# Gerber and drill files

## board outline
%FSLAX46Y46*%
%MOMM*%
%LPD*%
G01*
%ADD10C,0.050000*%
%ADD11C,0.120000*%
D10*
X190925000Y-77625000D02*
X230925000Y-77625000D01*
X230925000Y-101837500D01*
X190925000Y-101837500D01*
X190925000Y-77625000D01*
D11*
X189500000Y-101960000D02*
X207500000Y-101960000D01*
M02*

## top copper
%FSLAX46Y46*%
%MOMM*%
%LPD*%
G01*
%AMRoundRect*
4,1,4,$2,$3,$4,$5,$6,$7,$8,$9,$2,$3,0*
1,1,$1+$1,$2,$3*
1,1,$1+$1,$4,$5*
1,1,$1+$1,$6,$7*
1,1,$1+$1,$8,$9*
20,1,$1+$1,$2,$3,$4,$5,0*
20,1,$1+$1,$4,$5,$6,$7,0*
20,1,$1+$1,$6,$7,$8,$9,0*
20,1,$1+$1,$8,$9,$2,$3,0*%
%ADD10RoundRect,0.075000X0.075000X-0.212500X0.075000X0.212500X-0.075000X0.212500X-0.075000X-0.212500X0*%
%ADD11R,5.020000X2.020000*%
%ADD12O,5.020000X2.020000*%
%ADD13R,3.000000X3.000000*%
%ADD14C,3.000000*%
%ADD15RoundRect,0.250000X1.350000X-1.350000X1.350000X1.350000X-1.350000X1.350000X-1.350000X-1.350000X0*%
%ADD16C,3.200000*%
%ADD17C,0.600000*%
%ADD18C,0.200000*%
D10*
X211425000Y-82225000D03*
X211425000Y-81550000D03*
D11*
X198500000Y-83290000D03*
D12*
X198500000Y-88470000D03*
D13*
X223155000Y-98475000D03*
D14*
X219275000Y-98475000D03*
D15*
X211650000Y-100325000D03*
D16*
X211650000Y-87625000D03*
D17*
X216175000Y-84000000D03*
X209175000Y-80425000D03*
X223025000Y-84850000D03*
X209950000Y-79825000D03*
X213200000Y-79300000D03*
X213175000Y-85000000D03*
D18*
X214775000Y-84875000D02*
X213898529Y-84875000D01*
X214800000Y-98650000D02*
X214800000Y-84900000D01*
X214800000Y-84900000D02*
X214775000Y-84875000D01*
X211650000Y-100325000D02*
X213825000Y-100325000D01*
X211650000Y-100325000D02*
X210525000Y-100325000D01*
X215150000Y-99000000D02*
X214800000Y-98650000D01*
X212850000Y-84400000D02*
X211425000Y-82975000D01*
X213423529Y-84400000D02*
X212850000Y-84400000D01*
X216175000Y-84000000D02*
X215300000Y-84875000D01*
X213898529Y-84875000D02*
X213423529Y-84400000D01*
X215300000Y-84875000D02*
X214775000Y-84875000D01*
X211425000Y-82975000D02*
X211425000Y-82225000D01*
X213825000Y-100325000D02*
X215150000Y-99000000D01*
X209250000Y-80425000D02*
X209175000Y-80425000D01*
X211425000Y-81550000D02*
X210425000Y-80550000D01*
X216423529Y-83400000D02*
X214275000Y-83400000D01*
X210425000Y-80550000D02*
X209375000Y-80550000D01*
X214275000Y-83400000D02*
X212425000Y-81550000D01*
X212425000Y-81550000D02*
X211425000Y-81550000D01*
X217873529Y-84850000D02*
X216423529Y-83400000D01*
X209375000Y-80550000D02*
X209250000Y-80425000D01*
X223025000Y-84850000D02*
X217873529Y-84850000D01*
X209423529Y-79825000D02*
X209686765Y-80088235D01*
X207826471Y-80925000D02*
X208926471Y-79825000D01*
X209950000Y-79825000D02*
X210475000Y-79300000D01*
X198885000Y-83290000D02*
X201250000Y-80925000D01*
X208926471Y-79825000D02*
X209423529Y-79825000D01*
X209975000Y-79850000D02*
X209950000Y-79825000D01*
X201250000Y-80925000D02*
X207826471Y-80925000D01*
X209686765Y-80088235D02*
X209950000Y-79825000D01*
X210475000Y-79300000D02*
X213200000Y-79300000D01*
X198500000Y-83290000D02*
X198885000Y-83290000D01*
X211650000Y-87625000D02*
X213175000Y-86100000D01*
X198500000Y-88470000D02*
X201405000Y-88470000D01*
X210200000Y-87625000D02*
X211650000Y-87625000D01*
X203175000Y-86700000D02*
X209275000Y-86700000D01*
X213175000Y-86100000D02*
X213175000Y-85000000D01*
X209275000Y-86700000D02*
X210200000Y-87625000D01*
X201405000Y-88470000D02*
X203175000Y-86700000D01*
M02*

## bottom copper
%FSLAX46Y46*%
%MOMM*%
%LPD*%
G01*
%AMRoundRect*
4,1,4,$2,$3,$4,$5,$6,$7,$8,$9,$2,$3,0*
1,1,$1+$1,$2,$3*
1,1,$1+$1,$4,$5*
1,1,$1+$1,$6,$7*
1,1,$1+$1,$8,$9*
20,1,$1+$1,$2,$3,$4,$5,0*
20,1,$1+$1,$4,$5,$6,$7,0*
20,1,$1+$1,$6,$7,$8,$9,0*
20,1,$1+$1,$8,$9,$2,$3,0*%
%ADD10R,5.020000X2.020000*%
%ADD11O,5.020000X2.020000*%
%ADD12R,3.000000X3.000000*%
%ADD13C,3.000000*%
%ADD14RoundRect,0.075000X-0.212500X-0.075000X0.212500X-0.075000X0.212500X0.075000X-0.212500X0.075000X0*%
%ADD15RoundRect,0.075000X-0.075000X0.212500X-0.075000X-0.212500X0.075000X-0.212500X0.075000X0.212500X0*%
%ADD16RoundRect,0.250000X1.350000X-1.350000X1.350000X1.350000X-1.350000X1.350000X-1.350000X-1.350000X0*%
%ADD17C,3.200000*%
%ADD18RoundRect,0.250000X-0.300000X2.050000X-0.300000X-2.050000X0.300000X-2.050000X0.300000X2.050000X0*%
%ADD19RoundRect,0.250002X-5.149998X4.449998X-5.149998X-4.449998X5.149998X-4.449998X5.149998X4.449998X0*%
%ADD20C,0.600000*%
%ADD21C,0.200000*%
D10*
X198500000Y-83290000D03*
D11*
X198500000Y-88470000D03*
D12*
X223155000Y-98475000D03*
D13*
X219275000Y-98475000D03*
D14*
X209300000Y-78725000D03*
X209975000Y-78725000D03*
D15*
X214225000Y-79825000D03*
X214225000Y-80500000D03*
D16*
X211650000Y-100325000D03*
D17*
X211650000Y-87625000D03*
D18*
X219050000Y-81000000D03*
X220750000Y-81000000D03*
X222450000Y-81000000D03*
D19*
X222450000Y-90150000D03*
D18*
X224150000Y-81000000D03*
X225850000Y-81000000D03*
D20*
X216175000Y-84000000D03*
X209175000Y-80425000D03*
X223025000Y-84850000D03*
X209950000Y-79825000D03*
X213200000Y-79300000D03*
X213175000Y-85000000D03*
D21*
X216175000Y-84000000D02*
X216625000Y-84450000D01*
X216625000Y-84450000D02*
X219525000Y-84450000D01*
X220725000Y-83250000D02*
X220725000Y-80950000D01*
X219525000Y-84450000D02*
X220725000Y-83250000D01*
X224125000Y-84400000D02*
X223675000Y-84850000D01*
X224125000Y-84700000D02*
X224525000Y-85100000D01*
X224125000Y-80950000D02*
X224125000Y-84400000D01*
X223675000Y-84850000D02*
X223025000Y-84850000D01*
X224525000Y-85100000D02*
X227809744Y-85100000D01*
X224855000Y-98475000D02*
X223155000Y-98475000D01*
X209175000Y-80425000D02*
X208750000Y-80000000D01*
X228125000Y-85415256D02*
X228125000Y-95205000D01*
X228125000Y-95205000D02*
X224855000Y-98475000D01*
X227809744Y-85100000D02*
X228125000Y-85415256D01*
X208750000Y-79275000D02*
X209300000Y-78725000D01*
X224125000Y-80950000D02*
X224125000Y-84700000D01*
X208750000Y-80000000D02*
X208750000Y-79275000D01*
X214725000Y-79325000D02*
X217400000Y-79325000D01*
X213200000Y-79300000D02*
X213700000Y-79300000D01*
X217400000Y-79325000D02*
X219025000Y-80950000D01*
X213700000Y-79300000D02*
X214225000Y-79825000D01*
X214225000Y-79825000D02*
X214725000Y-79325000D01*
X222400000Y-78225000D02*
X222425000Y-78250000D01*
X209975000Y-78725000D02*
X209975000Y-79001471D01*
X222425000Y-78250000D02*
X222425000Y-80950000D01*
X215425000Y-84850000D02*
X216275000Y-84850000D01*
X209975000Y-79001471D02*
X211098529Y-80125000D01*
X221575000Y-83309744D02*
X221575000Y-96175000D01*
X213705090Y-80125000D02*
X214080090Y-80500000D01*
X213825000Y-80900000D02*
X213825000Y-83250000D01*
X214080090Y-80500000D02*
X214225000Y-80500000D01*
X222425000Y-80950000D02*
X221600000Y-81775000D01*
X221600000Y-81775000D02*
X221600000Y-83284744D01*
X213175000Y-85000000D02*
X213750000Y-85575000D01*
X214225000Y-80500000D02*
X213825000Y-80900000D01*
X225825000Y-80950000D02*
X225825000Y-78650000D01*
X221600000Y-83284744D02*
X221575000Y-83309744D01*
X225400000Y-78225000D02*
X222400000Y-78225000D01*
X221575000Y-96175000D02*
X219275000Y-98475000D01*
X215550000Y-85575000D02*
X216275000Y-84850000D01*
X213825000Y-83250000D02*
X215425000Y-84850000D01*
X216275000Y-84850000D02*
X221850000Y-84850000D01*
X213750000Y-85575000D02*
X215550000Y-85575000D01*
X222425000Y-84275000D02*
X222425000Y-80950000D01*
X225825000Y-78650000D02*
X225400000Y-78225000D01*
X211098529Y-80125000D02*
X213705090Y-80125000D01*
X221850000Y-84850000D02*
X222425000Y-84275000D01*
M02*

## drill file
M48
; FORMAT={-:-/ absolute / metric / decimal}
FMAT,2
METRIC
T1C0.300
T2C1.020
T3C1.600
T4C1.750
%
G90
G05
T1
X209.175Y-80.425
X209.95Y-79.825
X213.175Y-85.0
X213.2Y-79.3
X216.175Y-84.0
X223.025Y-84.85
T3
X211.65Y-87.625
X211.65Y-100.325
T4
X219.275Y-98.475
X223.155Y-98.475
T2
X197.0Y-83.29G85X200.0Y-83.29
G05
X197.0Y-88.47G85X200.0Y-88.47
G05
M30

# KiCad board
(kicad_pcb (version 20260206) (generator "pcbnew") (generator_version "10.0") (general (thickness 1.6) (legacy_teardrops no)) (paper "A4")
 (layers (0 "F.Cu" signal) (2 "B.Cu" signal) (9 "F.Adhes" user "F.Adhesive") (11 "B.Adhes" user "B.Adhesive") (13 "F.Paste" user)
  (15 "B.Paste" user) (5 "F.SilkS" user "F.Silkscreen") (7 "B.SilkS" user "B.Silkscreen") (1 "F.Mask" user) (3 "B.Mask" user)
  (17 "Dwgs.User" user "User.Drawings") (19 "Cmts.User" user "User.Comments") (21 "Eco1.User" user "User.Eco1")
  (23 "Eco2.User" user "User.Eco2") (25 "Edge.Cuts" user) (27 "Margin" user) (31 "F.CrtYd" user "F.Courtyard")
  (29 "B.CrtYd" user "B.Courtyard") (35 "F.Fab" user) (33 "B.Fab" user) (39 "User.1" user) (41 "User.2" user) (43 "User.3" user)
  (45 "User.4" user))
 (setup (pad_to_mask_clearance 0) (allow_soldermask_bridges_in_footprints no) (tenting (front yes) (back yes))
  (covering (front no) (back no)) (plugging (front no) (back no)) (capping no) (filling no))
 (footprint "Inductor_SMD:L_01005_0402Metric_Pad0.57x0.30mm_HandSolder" (layer "F.Cu") (at 211.425 81.8875 90)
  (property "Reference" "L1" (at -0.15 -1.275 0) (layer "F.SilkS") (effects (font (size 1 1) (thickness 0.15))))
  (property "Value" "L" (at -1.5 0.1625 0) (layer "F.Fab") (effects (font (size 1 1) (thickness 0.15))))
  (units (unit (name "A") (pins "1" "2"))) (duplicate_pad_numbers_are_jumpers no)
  (pad "" smd roundrect (at -0.3625 0 90) (size 0.41 0.27) (layers "F.Paste") (roundrect_rratio 0.25))
  (pad "" smd roundrect (at 0.3625 0 90) (size 0.41 0.27) (layers "F.Paste") (roundrect_rratio 0.25))
  (pad "1" smd roundrect (at -0.3375 0 90) (size 0.575 0.3) (layers "F.Cu" "F.Mask") (roundrect_rratio 0.25) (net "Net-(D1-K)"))
  (pad "2" smd roundrect (at 0.3375 0 90) (size 0.575 0.3) (layers "F.Cu" "F.Mask") (roundrect_rratio 0.25) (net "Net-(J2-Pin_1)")))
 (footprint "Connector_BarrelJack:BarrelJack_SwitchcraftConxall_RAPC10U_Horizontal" (layer "F.Cu") (at 198.5 83.29 90)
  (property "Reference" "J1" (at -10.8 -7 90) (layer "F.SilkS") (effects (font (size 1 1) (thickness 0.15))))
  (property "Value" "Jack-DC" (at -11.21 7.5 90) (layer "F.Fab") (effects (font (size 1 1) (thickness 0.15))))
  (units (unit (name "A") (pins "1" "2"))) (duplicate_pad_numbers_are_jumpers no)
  (fp_line (start -18.67 -9) (end -18.67 9) (stroke (width 0.12) (type solid)) (layer "Edge.Cuts"))
  (pad "1" thru_hole rect (at 0 0 90) (size 2.02 5.02) (drill oval 1.02 4.02) (layers "*.Cu" "*.Mask") (remove_unused_layers no)
   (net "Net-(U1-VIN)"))
  (pad "2" thru_hole oval (at -5.18 0 90) (size 2.02 5.02) (drill oval 1.02 4.02) (layers "*.Cu" "*.Mask") (remove_unused_layers no)
   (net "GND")))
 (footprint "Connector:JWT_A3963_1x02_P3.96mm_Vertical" (layer "F.Cu") (at 223.155 98.475 180)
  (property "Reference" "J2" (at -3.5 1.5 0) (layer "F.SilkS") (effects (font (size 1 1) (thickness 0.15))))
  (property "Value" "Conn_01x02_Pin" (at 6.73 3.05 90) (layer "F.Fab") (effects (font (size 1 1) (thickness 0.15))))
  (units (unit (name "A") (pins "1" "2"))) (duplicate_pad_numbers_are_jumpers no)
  (pad "1" thru_hole rect (at 0 0 180) (size 3 3) (drill 1.75) (layers "*.Cu" "*.Mask") (remove_unused_layers no) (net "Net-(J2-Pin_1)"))
  (pad "2" thru_hole circle (at 3.88 0 180) (size 3 3) (drill 1.75) (layers "*.Cu" "*.Mask") (remove_unused_layers no) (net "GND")))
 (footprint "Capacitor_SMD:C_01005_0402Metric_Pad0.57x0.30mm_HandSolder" (layer "B.Cu") (at 209.6375 78.725)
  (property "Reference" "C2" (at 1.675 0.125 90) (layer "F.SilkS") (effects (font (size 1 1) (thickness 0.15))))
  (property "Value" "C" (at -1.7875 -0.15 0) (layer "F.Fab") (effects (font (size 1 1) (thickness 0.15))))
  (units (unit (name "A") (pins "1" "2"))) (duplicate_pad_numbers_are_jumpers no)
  (pad "" smd roundrect (at -0.3625 0) (size 0.41 0.27) (layers "B.Paste") (roundrect_rratio 0.25))
  (pad "" smd roundrect (at 0.3625 0) (size 0.41 0.27) (layers "B.Paste") (roundrect_rratio 0.25))
  (pad "1" smd roundrect (at -0.3375 0) (size 0.575 0.3) (layers "B.Cu" "B.Mask") (roundrect_rratio 0.25) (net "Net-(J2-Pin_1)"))
  (pad "2" smd roundrect (at 0.3375 0) (size 0.575 0.3) (layers "B.Cu" "B.Mask") (roundrect_rratio 0.25) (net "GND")))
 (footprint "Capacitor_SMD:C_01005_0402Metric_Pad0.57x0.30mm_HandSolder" (layer "B.Cu") (at 214.225 80.1625 -90)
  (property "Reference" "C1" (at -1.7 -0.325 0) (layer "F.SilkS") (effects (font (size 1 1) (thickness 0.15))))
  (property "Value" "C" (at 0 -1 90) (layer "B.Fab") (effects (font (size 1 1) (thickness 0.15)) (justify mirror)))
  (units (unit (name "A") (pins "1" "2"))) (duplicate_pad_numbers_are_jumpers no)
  (pad "" smd roundrect (at -0.3625 0 270) (size 0.41 0.27) (layers "B.Paste") (roundrect_rratio 0.25))
  (pad "" smd roundrect (at 0.3625 0 270) (size 0.41 0.27) (layers "B.Paste") (roundrect_rratio 0.25))
  (pad "1" smd roundrect (at -0.3375 0 270) (size 0.575 0.3) (layers "B.Cu" "B.Mask") (roundrect_rratio 0.25) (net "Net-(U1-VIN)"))
  (pad "2" smd roundrect (at 0.3375 0 270) (size 0.575 0.3) (layers "B.Cu" "B.Mask") (roundrect_rratio 0.25) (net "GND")))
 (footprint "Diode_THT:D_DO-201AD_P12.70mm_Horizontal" (layer "B.Cu") (at 211.65 100.325 90)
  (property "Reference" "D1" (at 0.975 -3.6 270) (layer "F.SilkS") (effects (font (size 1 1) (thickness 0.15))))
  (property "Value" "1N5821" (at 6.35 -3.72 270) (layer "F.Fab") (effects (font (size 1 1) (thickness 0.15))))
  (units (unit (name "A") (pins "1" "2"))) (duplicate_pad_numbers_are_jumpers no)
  (pad "1" thru_hole roundrect (at 0 0 90) (size 3.2 3.2) (drill 1.6) (layers "*.Cu" "*.Mask") (remove_unused_layers no)
   (roundrect_rratio 0.078125) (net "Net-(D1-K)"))
  (pad "2" thru_hole circle (at 12.7 0 90) (size 3.2 3.2) (drill 1.6) (layers "*.Cu" "*.Mask") (remove_unused_layers no) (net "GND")))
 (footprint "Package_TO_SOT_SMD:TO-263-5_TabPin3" (layer "B.Cu") (at 222.45 88.65 -90)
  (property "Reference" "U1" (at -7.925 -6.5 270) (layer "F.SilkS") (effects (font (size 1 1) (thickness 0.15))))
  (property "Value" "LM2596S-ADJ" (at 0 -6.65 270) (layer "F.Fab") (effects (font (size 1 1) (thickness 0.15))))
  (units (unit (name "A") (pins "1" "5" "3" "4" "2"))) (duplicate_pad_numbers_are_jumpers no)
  (pad "" smd roundrect (at -0.925 -2.775 270) (size 4.55 5.25) (layers "B.Paste") (roundrect_rratio 0.054945))
  (pad "" smd roundrect (at -0.925 2.775 270) (size 4.55 5.25) (layers "B.Paste") (roundrect_rratio 0.054945))
  (pad "" smd roundrect (at 3.925 -2.775 270) (size 4.55 5.25) (layers "B.Paste") (roundrect_rratio 0.054945))
  (pad "" smd roundrect (at 3.925 2.775 270) (size 4.55 5.25) (layers "B.Paste") (roundrect_rratio 0.054945))
  (pad "1" smd roundrect (at -7.65 3.4 270) (size 4.6 1.1) (layers "B.Cu" "B.Mask" "B.Paste") (roundrect_rratio 0.227273)
   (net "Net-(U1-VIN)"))
  (pad "2" smd roundrect (at -7.65 1.7 270) (size 4.6 1.1) (layers "B.Cu" "B.Mask" "B.Paste") (roundrect_rratio 0.227273) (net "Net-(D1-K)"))
  (pad "3" smd roundrect (at -7.65 0 270) (size 4.6 1.1) (layers "B.Cu" "B.Mask" "B.Paste") (roundrect_rratio 0.227273) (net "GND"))
  (pad "3" smd roundrect (at 1.5 0 270) (size 9.4 10.8) (layers "B.Cu" "B.Mask") (roundrect_rratio 0.026596) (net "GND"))
  (pad "4" smd roundrect (at -7.65 -1.7 270) (size 4.6 1.1) (layers "B.Cu" "B.Mask" "B.Paste") (roundrect_rratio 0.227273)
   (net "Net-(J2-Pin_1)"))
  (pad "5" smd roundrect (at -7.65 -3.4 270) (size 4.6 1.1) (layers "B.Cu" "B.Mask" "B.Paste") (roundrect_rratio 0.227273) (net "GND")))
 (gr_rect (start 190.925 77.625) (end 230.925 101.8375) (stroke (width 0.05) (type default)) (fill no) (layer "Edge.Cuts"))
 (segment (start 214.775 84.875) (end 213.898529 84.875) (width 0.2) (layer "F.Cu") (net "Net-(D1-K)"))
 (segment (start 214.8 98.65) (end 214.8 84.9) (width 0.2) (layer "F.Cu") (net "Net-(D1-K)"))
 (segment (start 214.8 84.9) (end 214.775 84.875) (width 0.2) (layer "F.Cu") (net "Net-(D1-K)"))
 (segment (start 211.65 100.325) (end 213.825 100.325) (width 0.2) (layer "F.Cu") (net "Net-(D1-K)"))
 (segment (start 211.65 100.325) (end 210.525 100.325) (width 0.2) (layer "F.Cu") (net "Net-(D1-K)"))
 (segment (start 215.15 99) (end 214.8 98.65) (width 0.2) (layer "F.Cu") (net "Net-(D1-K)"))
 (segment (start 212.85 84.4) (end 211.425 82.975) (width 0.2) (layer "F.Cu") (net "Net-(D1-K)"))
 (segment (start 213.423529 84.4) (end 212.85 84.4) (width 0.2) (layer "F.Cu") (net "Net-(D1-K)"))
 (segment (start 216.175 84) (end 215.3 84.875) (width 0.2) (layer "F.Cu") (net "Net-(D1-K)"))
 (segment (start 213.898529 84.875) (end 213.423529 84.4) (width 0.2) (layer "F.Cu") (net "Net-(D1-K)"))
 (segment (start 215.3 84.875) (end 214.775 84.875) (width 0.2) (layer "F.Cu") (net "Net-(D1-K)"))
 (segment (start 211.425 82.975) (end 211.425 82.225) (width 0.2) (layer "F.Cu") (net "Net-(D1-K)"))
 (segment (start 213.825 100.325) (end 215.15 99) (width 0.2) (layer "F.Cu") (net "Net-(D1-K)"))
 (via (at 216.175 84) (size 0.6) (drill 0.3) (layers "F.Cu" "B.Cu") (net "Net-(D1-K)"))
 (segment (start 216.175 84) (end 216.625 84.45) (width 0.2) (layer "B.Cu") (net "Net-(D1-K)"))
 (segment (start 216.625 84.45) (end 219.525 84.45) (width 0.2) (layer "B.Cu") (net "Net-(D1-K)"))
 (segment (start 220.725 83.25) (end 220.725 80.95) (width 0.2) (layer "B.Cu") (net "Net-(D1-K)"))
 (segment (start 219.525 84.45) (end 220.725 83.25) (width 0.2) (layer "B.Cu") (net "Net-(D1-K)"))
 (segment (start 209.25 80.425) (end 209.175 80.425) (width 0.2) (layer "F.Cu") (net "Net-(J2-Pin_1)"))
 (segment (start 211.425 81.55) (end 210.425 80.55) (width 0.2) (layer "F.Cu") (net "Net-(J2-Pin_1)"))
 (segment (start 216.423529 83.4) (end 214.275 83.4) (width 0.2) (layer "F.Cu") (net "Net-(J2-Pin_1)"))
 (segment (start 210.425 80.55) (end 209.375 80.55) (width 0.2) (layer "F.Cu") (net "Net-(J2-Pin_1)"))
 (segment (start 214.275 83.4) (end 212.425 81.55) (width 0.2) (layer "F.Cu") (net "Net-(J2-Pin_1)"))
 (segment (start 212.425 81.55) (end 211.425 81.55) (width 0.2) (layer "F.Cu") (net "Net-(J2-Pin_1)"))
 (segment (start 217.873529 84.85) (end 216.423529 83.4) (width 0.2) (layer "F.Cu") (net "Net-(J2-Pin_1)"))
 (segment (start 209.375 80.55) (end 209.25 80.425) (width 0.2) (layer "F.Cu") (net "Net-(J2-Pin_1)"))
 (segment (start 223.025 84.85) (end 217.873529 84.85) (width 0.2) (layer "F.Cu") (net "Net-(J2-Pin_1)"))
 (via (at 209.175 80.425) (size 0.6) (drill 0.3) (layers "F.Cu" "B.Cu") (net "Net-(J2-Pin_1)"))
 (via (at 223.025 84.85) (size 0.6) (drill 0.3) (layers "F.Cu" "B.Cu") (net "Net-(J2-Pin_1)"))
 (segment (start 224.125 84.4) (end 223.675 84.85) (width 0.2) (layer "B.Cu") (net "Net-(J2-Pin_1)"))
 (segment (start 224.125 84.7) (end 224.525 85.1) (width 0.2) (layer "B.Cu") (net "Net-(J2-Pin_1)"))
 (segment (start 224.125 80.95) (end 224.125 84.4) (width 0.2) (layer "B.Cu") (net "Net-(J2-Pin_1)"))
 (segment (start 223.675 84.85) (end 223.025 84.85) (width 0.2) (layer "B.Cu") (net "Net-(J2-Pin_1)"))
 (segment (start 224.525 85.1) (end 227.809744 85.1) (width 0.2) (layer "B.Cu") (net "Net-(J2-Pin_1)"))
 (segment (start 224.855 98.475) (end 223.155 98.475) (width 0.2) (layer "B.Cu") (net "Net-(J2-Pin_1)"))
 (segment (start 209.175 80.425) (end 208.75 80) (width 0.2) (layer "B.Cu") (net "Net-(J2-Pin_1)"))
 (segment (start 228.125 85.415256) (end 228.125 95.205) (width 0.2) (layer "B.Cu") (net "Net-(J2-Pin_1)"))
 (segment (start 228.125 95.205) (end 224.855 98.475) (width 0.2) (layer "B.Cu") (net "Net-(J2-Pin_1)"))
 (segment (start 227.809744 85.1) (end 228.125 85.415256) (width 0.2) (layer "B.Cu") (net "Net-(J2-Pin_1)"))
 (segment (start 208.75 79.275) (end 209.3 78.725) (width 0.2) (layer "B.Cu") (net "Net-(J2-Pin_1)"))
 (segment (start 224.125 80.95) (end 224.125 84.7) (width 0.2) (layer "B.Cu") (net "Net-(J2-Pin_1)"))
 (segment (start 208.75 80) (end 208.75 79.275) (width 0.2) (layer "B.Cu") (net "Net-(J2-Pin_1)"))
 (segment (start 209.423529 79.825) (end 209.686765 80.088235) (width 0.2) (layer "F.Cu") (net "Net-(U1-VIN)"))
 (segment (start 207.826471 80.925) (end 208.926471 79.825) (width 0.2) (layer "F.Cu") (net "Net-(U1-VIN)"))
 (segment (start 209.95 79.825) (end 210.475 79.3) (width 0.2) (layer "F.Cu") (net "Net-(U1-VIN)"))
 (segment (start 198.885 83.29) (end 201.25 80.925) (width 0.2) (layer "F.Cu") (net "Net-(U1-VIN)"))
 (segment (start 208.926471 79.825) (end 209.423529 79.825) (width 0.2) (layer "F.Cu") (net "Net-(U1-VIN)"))
 (segment (start 209.975 79.85) (end 209.95 79.825) (width 0.2) (layer "F.Cu") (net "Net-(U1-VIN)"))
 (segment (start 201.25 80.925) (end 207.826471 80.925) (width 0.2) (layer "F.Cu") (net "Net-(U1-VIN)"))
 (segment (start 209.686765 80.088235) (end 209.95 79.825) (width 0.2) (layer "F.Cu") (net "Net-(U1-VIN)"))
 (segment (start 210.475 79.3) (end 213.2 79.3) (width 0.2) (layer "F.Cu") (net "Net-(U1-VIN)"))
 (segment (start 198.5 83.29) (end 198.885 83.29) (width 0.2) (layer "F.Cu") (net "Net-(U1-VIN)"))
 (via (at 209.95 79.825) (size 0.6) (drill 0.3) (layers "F.Cu" "B.Cu") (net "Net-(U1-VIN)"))
 (via (at 213.2 79.3) (size 0.6) (drill 0.3) (layers "F.Cu" "B.Cu") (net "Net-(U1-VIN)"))
 (segment (start 214.725 79.325) (end 217.4 79.325) (width 0.2) (layer "B.Cu") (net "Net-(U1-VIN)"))
 (segment (start 213.2 79.3) (end 213.7 79.3) (width 0.2) (layer "B.Cu") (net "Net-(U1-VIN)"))
 (segment (start 217.4 79.325) (end 219.025 80.95) (width 0.2) (layer "B.Cu") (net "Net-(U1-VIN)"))
 (segment (start 213.7 79.3) (end 214.225 79.825) (width 0.2) (layer "B.Cu") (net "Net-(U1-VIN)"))
 (segment (start 214.225 79.825) (end 214.725 79.325) (width 0.2) (layer "B.Cu") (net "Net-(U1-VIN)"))
 (segment (start 211.65 87.625) (end 213.175 86.1) (width 0.2) (layer "F.Cu") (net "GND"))
 (segment (start 198.5 88.47) (end 201.405 88.47) (width 0.2) (layer "F.Cu") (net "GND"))
 (segment (start 210.2 87.625) (end 211.65 87.625) (width 0.2) (layer "F.Cu") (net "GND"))
 (segment (start 203.175 86.7) (end 209.275 86.7) (width 0.2) (layer "F.Cu") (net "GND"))
 (segment (start 213.175 86.1) (end 213.175 85) (width 0.2) (layer "F.Cu") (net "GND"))
 (segment (start 209.275 86.7) (end 210.2 87.625) (width 0.2) (layer "F.Cu") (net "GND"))
 (segment (start 201.405 88.47) (end 203.175 86.7) (width 0.2) (layer "F.Cu") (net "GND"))
 (via (at 213.175 85) (size 0.6) (drill 0.3) (layers "F.Cu" "B.Cu") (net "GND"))
 (segment (start 222.4 78.225) (end 222.425 78.25) (width 0.2) (layer "B.Cu") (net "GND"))
 (segment (start 209.975 78.725) (end 209.975 79.001471) (width 0.2) (layer "B.Cu") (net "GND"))
 (segment (start 222.425 78.25) (end 222.425 80.95) (width 0.2) (layer "B.Cu") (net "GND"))
 (segment (start 215.425 84.85) (end 216.275 84.85) (width 0.2) (layer "B.Cu") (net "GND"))
 (segment (start 209.975 79.001471) (end 211.098529 80.125) (width 0.2) (layer "B.Cu") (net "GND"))
 (segment (start 221.575 83.309744) (end 221.575 96.175) (width 0.2) (layer "B.Cu") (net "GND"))
 (segment (start 213.70509 80.125) (end 214.08009 80.5) (width 0.2) (layer "B.Cu") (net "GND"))
 (segment (start 213.825 80.9) (end 213.825 83.25) (width 0.2) (layer "B.Cu") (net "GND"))
 (segment (start 214.08009 80.5) (end 214.225 80.5) (width 0.2) (layer "B.Cu") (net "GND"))
 (segment (start 222.425 80.95) (end 221.6 81.775) (width 0.2) (layer "B.Cu") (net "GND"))
 (segment (start 221.6 81.775) (end 221.6 83.284744) (width 0.2) (layer "B.Cu") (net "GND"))
 (segment (start 213.175 85) (end 213.75 85.575) (width 0.2) (layer "B.Cu") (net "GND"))
 (segment (start 214.225 80.5) (end 213.825 80.9) (width 0.2) (layer "B.Cu") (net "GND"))
 (segment (start 225.825 80.95) (end 225.825 78.65) (width 0.2) (layer "B.Cu") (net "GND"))
 (segment (start 221.6 83.284744) (end 221.575 83.309744) (width 0.2) (layer "B.Cu") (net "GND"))
 (segment (start 225.4 78.225) (end 222.4 78.225) (width 0.2) (layer "B.Cu") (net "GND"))
 (segment (start 221.575 96.175) (end 219.275 98.475) (width 0.2) (layer "B.Cu") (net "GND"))
 (segment (start 215.55 85.575) (end 216.275 84.85) (width 0.2) (layer "B.Cu") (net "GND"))
 (segment (start 213.825 83.25) (end 215.425 84.85) (width 0.2) (layer "B.Cu") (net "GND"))
 (segment (start 216.275 84.85) (end 221.85 84.85) (width 0.2) (layer "B.Cu") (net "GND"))
 (segment (start 213.75 85.575) (end 215.55 85.575) (width 0.2) (layer "B.Cu") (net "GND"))
 (segment (start 222.425 84.275) (end 222.425 80.95) (width 0.2) (layer "B.Cu") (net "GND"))
 (segment (start 225.825 78.65) (end 225.4 78.225) (width 0.2) (layer "B.Cu") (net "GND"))
 (segment (start 211.098529 80.125) (end 213.70509 80.125) (width 0.2) (layer "B.Cu") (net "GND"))
 (segment (start 221.85 84.85) (end 222.425 84.275) (width 0.2) (layer "B.Cu") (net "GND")))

